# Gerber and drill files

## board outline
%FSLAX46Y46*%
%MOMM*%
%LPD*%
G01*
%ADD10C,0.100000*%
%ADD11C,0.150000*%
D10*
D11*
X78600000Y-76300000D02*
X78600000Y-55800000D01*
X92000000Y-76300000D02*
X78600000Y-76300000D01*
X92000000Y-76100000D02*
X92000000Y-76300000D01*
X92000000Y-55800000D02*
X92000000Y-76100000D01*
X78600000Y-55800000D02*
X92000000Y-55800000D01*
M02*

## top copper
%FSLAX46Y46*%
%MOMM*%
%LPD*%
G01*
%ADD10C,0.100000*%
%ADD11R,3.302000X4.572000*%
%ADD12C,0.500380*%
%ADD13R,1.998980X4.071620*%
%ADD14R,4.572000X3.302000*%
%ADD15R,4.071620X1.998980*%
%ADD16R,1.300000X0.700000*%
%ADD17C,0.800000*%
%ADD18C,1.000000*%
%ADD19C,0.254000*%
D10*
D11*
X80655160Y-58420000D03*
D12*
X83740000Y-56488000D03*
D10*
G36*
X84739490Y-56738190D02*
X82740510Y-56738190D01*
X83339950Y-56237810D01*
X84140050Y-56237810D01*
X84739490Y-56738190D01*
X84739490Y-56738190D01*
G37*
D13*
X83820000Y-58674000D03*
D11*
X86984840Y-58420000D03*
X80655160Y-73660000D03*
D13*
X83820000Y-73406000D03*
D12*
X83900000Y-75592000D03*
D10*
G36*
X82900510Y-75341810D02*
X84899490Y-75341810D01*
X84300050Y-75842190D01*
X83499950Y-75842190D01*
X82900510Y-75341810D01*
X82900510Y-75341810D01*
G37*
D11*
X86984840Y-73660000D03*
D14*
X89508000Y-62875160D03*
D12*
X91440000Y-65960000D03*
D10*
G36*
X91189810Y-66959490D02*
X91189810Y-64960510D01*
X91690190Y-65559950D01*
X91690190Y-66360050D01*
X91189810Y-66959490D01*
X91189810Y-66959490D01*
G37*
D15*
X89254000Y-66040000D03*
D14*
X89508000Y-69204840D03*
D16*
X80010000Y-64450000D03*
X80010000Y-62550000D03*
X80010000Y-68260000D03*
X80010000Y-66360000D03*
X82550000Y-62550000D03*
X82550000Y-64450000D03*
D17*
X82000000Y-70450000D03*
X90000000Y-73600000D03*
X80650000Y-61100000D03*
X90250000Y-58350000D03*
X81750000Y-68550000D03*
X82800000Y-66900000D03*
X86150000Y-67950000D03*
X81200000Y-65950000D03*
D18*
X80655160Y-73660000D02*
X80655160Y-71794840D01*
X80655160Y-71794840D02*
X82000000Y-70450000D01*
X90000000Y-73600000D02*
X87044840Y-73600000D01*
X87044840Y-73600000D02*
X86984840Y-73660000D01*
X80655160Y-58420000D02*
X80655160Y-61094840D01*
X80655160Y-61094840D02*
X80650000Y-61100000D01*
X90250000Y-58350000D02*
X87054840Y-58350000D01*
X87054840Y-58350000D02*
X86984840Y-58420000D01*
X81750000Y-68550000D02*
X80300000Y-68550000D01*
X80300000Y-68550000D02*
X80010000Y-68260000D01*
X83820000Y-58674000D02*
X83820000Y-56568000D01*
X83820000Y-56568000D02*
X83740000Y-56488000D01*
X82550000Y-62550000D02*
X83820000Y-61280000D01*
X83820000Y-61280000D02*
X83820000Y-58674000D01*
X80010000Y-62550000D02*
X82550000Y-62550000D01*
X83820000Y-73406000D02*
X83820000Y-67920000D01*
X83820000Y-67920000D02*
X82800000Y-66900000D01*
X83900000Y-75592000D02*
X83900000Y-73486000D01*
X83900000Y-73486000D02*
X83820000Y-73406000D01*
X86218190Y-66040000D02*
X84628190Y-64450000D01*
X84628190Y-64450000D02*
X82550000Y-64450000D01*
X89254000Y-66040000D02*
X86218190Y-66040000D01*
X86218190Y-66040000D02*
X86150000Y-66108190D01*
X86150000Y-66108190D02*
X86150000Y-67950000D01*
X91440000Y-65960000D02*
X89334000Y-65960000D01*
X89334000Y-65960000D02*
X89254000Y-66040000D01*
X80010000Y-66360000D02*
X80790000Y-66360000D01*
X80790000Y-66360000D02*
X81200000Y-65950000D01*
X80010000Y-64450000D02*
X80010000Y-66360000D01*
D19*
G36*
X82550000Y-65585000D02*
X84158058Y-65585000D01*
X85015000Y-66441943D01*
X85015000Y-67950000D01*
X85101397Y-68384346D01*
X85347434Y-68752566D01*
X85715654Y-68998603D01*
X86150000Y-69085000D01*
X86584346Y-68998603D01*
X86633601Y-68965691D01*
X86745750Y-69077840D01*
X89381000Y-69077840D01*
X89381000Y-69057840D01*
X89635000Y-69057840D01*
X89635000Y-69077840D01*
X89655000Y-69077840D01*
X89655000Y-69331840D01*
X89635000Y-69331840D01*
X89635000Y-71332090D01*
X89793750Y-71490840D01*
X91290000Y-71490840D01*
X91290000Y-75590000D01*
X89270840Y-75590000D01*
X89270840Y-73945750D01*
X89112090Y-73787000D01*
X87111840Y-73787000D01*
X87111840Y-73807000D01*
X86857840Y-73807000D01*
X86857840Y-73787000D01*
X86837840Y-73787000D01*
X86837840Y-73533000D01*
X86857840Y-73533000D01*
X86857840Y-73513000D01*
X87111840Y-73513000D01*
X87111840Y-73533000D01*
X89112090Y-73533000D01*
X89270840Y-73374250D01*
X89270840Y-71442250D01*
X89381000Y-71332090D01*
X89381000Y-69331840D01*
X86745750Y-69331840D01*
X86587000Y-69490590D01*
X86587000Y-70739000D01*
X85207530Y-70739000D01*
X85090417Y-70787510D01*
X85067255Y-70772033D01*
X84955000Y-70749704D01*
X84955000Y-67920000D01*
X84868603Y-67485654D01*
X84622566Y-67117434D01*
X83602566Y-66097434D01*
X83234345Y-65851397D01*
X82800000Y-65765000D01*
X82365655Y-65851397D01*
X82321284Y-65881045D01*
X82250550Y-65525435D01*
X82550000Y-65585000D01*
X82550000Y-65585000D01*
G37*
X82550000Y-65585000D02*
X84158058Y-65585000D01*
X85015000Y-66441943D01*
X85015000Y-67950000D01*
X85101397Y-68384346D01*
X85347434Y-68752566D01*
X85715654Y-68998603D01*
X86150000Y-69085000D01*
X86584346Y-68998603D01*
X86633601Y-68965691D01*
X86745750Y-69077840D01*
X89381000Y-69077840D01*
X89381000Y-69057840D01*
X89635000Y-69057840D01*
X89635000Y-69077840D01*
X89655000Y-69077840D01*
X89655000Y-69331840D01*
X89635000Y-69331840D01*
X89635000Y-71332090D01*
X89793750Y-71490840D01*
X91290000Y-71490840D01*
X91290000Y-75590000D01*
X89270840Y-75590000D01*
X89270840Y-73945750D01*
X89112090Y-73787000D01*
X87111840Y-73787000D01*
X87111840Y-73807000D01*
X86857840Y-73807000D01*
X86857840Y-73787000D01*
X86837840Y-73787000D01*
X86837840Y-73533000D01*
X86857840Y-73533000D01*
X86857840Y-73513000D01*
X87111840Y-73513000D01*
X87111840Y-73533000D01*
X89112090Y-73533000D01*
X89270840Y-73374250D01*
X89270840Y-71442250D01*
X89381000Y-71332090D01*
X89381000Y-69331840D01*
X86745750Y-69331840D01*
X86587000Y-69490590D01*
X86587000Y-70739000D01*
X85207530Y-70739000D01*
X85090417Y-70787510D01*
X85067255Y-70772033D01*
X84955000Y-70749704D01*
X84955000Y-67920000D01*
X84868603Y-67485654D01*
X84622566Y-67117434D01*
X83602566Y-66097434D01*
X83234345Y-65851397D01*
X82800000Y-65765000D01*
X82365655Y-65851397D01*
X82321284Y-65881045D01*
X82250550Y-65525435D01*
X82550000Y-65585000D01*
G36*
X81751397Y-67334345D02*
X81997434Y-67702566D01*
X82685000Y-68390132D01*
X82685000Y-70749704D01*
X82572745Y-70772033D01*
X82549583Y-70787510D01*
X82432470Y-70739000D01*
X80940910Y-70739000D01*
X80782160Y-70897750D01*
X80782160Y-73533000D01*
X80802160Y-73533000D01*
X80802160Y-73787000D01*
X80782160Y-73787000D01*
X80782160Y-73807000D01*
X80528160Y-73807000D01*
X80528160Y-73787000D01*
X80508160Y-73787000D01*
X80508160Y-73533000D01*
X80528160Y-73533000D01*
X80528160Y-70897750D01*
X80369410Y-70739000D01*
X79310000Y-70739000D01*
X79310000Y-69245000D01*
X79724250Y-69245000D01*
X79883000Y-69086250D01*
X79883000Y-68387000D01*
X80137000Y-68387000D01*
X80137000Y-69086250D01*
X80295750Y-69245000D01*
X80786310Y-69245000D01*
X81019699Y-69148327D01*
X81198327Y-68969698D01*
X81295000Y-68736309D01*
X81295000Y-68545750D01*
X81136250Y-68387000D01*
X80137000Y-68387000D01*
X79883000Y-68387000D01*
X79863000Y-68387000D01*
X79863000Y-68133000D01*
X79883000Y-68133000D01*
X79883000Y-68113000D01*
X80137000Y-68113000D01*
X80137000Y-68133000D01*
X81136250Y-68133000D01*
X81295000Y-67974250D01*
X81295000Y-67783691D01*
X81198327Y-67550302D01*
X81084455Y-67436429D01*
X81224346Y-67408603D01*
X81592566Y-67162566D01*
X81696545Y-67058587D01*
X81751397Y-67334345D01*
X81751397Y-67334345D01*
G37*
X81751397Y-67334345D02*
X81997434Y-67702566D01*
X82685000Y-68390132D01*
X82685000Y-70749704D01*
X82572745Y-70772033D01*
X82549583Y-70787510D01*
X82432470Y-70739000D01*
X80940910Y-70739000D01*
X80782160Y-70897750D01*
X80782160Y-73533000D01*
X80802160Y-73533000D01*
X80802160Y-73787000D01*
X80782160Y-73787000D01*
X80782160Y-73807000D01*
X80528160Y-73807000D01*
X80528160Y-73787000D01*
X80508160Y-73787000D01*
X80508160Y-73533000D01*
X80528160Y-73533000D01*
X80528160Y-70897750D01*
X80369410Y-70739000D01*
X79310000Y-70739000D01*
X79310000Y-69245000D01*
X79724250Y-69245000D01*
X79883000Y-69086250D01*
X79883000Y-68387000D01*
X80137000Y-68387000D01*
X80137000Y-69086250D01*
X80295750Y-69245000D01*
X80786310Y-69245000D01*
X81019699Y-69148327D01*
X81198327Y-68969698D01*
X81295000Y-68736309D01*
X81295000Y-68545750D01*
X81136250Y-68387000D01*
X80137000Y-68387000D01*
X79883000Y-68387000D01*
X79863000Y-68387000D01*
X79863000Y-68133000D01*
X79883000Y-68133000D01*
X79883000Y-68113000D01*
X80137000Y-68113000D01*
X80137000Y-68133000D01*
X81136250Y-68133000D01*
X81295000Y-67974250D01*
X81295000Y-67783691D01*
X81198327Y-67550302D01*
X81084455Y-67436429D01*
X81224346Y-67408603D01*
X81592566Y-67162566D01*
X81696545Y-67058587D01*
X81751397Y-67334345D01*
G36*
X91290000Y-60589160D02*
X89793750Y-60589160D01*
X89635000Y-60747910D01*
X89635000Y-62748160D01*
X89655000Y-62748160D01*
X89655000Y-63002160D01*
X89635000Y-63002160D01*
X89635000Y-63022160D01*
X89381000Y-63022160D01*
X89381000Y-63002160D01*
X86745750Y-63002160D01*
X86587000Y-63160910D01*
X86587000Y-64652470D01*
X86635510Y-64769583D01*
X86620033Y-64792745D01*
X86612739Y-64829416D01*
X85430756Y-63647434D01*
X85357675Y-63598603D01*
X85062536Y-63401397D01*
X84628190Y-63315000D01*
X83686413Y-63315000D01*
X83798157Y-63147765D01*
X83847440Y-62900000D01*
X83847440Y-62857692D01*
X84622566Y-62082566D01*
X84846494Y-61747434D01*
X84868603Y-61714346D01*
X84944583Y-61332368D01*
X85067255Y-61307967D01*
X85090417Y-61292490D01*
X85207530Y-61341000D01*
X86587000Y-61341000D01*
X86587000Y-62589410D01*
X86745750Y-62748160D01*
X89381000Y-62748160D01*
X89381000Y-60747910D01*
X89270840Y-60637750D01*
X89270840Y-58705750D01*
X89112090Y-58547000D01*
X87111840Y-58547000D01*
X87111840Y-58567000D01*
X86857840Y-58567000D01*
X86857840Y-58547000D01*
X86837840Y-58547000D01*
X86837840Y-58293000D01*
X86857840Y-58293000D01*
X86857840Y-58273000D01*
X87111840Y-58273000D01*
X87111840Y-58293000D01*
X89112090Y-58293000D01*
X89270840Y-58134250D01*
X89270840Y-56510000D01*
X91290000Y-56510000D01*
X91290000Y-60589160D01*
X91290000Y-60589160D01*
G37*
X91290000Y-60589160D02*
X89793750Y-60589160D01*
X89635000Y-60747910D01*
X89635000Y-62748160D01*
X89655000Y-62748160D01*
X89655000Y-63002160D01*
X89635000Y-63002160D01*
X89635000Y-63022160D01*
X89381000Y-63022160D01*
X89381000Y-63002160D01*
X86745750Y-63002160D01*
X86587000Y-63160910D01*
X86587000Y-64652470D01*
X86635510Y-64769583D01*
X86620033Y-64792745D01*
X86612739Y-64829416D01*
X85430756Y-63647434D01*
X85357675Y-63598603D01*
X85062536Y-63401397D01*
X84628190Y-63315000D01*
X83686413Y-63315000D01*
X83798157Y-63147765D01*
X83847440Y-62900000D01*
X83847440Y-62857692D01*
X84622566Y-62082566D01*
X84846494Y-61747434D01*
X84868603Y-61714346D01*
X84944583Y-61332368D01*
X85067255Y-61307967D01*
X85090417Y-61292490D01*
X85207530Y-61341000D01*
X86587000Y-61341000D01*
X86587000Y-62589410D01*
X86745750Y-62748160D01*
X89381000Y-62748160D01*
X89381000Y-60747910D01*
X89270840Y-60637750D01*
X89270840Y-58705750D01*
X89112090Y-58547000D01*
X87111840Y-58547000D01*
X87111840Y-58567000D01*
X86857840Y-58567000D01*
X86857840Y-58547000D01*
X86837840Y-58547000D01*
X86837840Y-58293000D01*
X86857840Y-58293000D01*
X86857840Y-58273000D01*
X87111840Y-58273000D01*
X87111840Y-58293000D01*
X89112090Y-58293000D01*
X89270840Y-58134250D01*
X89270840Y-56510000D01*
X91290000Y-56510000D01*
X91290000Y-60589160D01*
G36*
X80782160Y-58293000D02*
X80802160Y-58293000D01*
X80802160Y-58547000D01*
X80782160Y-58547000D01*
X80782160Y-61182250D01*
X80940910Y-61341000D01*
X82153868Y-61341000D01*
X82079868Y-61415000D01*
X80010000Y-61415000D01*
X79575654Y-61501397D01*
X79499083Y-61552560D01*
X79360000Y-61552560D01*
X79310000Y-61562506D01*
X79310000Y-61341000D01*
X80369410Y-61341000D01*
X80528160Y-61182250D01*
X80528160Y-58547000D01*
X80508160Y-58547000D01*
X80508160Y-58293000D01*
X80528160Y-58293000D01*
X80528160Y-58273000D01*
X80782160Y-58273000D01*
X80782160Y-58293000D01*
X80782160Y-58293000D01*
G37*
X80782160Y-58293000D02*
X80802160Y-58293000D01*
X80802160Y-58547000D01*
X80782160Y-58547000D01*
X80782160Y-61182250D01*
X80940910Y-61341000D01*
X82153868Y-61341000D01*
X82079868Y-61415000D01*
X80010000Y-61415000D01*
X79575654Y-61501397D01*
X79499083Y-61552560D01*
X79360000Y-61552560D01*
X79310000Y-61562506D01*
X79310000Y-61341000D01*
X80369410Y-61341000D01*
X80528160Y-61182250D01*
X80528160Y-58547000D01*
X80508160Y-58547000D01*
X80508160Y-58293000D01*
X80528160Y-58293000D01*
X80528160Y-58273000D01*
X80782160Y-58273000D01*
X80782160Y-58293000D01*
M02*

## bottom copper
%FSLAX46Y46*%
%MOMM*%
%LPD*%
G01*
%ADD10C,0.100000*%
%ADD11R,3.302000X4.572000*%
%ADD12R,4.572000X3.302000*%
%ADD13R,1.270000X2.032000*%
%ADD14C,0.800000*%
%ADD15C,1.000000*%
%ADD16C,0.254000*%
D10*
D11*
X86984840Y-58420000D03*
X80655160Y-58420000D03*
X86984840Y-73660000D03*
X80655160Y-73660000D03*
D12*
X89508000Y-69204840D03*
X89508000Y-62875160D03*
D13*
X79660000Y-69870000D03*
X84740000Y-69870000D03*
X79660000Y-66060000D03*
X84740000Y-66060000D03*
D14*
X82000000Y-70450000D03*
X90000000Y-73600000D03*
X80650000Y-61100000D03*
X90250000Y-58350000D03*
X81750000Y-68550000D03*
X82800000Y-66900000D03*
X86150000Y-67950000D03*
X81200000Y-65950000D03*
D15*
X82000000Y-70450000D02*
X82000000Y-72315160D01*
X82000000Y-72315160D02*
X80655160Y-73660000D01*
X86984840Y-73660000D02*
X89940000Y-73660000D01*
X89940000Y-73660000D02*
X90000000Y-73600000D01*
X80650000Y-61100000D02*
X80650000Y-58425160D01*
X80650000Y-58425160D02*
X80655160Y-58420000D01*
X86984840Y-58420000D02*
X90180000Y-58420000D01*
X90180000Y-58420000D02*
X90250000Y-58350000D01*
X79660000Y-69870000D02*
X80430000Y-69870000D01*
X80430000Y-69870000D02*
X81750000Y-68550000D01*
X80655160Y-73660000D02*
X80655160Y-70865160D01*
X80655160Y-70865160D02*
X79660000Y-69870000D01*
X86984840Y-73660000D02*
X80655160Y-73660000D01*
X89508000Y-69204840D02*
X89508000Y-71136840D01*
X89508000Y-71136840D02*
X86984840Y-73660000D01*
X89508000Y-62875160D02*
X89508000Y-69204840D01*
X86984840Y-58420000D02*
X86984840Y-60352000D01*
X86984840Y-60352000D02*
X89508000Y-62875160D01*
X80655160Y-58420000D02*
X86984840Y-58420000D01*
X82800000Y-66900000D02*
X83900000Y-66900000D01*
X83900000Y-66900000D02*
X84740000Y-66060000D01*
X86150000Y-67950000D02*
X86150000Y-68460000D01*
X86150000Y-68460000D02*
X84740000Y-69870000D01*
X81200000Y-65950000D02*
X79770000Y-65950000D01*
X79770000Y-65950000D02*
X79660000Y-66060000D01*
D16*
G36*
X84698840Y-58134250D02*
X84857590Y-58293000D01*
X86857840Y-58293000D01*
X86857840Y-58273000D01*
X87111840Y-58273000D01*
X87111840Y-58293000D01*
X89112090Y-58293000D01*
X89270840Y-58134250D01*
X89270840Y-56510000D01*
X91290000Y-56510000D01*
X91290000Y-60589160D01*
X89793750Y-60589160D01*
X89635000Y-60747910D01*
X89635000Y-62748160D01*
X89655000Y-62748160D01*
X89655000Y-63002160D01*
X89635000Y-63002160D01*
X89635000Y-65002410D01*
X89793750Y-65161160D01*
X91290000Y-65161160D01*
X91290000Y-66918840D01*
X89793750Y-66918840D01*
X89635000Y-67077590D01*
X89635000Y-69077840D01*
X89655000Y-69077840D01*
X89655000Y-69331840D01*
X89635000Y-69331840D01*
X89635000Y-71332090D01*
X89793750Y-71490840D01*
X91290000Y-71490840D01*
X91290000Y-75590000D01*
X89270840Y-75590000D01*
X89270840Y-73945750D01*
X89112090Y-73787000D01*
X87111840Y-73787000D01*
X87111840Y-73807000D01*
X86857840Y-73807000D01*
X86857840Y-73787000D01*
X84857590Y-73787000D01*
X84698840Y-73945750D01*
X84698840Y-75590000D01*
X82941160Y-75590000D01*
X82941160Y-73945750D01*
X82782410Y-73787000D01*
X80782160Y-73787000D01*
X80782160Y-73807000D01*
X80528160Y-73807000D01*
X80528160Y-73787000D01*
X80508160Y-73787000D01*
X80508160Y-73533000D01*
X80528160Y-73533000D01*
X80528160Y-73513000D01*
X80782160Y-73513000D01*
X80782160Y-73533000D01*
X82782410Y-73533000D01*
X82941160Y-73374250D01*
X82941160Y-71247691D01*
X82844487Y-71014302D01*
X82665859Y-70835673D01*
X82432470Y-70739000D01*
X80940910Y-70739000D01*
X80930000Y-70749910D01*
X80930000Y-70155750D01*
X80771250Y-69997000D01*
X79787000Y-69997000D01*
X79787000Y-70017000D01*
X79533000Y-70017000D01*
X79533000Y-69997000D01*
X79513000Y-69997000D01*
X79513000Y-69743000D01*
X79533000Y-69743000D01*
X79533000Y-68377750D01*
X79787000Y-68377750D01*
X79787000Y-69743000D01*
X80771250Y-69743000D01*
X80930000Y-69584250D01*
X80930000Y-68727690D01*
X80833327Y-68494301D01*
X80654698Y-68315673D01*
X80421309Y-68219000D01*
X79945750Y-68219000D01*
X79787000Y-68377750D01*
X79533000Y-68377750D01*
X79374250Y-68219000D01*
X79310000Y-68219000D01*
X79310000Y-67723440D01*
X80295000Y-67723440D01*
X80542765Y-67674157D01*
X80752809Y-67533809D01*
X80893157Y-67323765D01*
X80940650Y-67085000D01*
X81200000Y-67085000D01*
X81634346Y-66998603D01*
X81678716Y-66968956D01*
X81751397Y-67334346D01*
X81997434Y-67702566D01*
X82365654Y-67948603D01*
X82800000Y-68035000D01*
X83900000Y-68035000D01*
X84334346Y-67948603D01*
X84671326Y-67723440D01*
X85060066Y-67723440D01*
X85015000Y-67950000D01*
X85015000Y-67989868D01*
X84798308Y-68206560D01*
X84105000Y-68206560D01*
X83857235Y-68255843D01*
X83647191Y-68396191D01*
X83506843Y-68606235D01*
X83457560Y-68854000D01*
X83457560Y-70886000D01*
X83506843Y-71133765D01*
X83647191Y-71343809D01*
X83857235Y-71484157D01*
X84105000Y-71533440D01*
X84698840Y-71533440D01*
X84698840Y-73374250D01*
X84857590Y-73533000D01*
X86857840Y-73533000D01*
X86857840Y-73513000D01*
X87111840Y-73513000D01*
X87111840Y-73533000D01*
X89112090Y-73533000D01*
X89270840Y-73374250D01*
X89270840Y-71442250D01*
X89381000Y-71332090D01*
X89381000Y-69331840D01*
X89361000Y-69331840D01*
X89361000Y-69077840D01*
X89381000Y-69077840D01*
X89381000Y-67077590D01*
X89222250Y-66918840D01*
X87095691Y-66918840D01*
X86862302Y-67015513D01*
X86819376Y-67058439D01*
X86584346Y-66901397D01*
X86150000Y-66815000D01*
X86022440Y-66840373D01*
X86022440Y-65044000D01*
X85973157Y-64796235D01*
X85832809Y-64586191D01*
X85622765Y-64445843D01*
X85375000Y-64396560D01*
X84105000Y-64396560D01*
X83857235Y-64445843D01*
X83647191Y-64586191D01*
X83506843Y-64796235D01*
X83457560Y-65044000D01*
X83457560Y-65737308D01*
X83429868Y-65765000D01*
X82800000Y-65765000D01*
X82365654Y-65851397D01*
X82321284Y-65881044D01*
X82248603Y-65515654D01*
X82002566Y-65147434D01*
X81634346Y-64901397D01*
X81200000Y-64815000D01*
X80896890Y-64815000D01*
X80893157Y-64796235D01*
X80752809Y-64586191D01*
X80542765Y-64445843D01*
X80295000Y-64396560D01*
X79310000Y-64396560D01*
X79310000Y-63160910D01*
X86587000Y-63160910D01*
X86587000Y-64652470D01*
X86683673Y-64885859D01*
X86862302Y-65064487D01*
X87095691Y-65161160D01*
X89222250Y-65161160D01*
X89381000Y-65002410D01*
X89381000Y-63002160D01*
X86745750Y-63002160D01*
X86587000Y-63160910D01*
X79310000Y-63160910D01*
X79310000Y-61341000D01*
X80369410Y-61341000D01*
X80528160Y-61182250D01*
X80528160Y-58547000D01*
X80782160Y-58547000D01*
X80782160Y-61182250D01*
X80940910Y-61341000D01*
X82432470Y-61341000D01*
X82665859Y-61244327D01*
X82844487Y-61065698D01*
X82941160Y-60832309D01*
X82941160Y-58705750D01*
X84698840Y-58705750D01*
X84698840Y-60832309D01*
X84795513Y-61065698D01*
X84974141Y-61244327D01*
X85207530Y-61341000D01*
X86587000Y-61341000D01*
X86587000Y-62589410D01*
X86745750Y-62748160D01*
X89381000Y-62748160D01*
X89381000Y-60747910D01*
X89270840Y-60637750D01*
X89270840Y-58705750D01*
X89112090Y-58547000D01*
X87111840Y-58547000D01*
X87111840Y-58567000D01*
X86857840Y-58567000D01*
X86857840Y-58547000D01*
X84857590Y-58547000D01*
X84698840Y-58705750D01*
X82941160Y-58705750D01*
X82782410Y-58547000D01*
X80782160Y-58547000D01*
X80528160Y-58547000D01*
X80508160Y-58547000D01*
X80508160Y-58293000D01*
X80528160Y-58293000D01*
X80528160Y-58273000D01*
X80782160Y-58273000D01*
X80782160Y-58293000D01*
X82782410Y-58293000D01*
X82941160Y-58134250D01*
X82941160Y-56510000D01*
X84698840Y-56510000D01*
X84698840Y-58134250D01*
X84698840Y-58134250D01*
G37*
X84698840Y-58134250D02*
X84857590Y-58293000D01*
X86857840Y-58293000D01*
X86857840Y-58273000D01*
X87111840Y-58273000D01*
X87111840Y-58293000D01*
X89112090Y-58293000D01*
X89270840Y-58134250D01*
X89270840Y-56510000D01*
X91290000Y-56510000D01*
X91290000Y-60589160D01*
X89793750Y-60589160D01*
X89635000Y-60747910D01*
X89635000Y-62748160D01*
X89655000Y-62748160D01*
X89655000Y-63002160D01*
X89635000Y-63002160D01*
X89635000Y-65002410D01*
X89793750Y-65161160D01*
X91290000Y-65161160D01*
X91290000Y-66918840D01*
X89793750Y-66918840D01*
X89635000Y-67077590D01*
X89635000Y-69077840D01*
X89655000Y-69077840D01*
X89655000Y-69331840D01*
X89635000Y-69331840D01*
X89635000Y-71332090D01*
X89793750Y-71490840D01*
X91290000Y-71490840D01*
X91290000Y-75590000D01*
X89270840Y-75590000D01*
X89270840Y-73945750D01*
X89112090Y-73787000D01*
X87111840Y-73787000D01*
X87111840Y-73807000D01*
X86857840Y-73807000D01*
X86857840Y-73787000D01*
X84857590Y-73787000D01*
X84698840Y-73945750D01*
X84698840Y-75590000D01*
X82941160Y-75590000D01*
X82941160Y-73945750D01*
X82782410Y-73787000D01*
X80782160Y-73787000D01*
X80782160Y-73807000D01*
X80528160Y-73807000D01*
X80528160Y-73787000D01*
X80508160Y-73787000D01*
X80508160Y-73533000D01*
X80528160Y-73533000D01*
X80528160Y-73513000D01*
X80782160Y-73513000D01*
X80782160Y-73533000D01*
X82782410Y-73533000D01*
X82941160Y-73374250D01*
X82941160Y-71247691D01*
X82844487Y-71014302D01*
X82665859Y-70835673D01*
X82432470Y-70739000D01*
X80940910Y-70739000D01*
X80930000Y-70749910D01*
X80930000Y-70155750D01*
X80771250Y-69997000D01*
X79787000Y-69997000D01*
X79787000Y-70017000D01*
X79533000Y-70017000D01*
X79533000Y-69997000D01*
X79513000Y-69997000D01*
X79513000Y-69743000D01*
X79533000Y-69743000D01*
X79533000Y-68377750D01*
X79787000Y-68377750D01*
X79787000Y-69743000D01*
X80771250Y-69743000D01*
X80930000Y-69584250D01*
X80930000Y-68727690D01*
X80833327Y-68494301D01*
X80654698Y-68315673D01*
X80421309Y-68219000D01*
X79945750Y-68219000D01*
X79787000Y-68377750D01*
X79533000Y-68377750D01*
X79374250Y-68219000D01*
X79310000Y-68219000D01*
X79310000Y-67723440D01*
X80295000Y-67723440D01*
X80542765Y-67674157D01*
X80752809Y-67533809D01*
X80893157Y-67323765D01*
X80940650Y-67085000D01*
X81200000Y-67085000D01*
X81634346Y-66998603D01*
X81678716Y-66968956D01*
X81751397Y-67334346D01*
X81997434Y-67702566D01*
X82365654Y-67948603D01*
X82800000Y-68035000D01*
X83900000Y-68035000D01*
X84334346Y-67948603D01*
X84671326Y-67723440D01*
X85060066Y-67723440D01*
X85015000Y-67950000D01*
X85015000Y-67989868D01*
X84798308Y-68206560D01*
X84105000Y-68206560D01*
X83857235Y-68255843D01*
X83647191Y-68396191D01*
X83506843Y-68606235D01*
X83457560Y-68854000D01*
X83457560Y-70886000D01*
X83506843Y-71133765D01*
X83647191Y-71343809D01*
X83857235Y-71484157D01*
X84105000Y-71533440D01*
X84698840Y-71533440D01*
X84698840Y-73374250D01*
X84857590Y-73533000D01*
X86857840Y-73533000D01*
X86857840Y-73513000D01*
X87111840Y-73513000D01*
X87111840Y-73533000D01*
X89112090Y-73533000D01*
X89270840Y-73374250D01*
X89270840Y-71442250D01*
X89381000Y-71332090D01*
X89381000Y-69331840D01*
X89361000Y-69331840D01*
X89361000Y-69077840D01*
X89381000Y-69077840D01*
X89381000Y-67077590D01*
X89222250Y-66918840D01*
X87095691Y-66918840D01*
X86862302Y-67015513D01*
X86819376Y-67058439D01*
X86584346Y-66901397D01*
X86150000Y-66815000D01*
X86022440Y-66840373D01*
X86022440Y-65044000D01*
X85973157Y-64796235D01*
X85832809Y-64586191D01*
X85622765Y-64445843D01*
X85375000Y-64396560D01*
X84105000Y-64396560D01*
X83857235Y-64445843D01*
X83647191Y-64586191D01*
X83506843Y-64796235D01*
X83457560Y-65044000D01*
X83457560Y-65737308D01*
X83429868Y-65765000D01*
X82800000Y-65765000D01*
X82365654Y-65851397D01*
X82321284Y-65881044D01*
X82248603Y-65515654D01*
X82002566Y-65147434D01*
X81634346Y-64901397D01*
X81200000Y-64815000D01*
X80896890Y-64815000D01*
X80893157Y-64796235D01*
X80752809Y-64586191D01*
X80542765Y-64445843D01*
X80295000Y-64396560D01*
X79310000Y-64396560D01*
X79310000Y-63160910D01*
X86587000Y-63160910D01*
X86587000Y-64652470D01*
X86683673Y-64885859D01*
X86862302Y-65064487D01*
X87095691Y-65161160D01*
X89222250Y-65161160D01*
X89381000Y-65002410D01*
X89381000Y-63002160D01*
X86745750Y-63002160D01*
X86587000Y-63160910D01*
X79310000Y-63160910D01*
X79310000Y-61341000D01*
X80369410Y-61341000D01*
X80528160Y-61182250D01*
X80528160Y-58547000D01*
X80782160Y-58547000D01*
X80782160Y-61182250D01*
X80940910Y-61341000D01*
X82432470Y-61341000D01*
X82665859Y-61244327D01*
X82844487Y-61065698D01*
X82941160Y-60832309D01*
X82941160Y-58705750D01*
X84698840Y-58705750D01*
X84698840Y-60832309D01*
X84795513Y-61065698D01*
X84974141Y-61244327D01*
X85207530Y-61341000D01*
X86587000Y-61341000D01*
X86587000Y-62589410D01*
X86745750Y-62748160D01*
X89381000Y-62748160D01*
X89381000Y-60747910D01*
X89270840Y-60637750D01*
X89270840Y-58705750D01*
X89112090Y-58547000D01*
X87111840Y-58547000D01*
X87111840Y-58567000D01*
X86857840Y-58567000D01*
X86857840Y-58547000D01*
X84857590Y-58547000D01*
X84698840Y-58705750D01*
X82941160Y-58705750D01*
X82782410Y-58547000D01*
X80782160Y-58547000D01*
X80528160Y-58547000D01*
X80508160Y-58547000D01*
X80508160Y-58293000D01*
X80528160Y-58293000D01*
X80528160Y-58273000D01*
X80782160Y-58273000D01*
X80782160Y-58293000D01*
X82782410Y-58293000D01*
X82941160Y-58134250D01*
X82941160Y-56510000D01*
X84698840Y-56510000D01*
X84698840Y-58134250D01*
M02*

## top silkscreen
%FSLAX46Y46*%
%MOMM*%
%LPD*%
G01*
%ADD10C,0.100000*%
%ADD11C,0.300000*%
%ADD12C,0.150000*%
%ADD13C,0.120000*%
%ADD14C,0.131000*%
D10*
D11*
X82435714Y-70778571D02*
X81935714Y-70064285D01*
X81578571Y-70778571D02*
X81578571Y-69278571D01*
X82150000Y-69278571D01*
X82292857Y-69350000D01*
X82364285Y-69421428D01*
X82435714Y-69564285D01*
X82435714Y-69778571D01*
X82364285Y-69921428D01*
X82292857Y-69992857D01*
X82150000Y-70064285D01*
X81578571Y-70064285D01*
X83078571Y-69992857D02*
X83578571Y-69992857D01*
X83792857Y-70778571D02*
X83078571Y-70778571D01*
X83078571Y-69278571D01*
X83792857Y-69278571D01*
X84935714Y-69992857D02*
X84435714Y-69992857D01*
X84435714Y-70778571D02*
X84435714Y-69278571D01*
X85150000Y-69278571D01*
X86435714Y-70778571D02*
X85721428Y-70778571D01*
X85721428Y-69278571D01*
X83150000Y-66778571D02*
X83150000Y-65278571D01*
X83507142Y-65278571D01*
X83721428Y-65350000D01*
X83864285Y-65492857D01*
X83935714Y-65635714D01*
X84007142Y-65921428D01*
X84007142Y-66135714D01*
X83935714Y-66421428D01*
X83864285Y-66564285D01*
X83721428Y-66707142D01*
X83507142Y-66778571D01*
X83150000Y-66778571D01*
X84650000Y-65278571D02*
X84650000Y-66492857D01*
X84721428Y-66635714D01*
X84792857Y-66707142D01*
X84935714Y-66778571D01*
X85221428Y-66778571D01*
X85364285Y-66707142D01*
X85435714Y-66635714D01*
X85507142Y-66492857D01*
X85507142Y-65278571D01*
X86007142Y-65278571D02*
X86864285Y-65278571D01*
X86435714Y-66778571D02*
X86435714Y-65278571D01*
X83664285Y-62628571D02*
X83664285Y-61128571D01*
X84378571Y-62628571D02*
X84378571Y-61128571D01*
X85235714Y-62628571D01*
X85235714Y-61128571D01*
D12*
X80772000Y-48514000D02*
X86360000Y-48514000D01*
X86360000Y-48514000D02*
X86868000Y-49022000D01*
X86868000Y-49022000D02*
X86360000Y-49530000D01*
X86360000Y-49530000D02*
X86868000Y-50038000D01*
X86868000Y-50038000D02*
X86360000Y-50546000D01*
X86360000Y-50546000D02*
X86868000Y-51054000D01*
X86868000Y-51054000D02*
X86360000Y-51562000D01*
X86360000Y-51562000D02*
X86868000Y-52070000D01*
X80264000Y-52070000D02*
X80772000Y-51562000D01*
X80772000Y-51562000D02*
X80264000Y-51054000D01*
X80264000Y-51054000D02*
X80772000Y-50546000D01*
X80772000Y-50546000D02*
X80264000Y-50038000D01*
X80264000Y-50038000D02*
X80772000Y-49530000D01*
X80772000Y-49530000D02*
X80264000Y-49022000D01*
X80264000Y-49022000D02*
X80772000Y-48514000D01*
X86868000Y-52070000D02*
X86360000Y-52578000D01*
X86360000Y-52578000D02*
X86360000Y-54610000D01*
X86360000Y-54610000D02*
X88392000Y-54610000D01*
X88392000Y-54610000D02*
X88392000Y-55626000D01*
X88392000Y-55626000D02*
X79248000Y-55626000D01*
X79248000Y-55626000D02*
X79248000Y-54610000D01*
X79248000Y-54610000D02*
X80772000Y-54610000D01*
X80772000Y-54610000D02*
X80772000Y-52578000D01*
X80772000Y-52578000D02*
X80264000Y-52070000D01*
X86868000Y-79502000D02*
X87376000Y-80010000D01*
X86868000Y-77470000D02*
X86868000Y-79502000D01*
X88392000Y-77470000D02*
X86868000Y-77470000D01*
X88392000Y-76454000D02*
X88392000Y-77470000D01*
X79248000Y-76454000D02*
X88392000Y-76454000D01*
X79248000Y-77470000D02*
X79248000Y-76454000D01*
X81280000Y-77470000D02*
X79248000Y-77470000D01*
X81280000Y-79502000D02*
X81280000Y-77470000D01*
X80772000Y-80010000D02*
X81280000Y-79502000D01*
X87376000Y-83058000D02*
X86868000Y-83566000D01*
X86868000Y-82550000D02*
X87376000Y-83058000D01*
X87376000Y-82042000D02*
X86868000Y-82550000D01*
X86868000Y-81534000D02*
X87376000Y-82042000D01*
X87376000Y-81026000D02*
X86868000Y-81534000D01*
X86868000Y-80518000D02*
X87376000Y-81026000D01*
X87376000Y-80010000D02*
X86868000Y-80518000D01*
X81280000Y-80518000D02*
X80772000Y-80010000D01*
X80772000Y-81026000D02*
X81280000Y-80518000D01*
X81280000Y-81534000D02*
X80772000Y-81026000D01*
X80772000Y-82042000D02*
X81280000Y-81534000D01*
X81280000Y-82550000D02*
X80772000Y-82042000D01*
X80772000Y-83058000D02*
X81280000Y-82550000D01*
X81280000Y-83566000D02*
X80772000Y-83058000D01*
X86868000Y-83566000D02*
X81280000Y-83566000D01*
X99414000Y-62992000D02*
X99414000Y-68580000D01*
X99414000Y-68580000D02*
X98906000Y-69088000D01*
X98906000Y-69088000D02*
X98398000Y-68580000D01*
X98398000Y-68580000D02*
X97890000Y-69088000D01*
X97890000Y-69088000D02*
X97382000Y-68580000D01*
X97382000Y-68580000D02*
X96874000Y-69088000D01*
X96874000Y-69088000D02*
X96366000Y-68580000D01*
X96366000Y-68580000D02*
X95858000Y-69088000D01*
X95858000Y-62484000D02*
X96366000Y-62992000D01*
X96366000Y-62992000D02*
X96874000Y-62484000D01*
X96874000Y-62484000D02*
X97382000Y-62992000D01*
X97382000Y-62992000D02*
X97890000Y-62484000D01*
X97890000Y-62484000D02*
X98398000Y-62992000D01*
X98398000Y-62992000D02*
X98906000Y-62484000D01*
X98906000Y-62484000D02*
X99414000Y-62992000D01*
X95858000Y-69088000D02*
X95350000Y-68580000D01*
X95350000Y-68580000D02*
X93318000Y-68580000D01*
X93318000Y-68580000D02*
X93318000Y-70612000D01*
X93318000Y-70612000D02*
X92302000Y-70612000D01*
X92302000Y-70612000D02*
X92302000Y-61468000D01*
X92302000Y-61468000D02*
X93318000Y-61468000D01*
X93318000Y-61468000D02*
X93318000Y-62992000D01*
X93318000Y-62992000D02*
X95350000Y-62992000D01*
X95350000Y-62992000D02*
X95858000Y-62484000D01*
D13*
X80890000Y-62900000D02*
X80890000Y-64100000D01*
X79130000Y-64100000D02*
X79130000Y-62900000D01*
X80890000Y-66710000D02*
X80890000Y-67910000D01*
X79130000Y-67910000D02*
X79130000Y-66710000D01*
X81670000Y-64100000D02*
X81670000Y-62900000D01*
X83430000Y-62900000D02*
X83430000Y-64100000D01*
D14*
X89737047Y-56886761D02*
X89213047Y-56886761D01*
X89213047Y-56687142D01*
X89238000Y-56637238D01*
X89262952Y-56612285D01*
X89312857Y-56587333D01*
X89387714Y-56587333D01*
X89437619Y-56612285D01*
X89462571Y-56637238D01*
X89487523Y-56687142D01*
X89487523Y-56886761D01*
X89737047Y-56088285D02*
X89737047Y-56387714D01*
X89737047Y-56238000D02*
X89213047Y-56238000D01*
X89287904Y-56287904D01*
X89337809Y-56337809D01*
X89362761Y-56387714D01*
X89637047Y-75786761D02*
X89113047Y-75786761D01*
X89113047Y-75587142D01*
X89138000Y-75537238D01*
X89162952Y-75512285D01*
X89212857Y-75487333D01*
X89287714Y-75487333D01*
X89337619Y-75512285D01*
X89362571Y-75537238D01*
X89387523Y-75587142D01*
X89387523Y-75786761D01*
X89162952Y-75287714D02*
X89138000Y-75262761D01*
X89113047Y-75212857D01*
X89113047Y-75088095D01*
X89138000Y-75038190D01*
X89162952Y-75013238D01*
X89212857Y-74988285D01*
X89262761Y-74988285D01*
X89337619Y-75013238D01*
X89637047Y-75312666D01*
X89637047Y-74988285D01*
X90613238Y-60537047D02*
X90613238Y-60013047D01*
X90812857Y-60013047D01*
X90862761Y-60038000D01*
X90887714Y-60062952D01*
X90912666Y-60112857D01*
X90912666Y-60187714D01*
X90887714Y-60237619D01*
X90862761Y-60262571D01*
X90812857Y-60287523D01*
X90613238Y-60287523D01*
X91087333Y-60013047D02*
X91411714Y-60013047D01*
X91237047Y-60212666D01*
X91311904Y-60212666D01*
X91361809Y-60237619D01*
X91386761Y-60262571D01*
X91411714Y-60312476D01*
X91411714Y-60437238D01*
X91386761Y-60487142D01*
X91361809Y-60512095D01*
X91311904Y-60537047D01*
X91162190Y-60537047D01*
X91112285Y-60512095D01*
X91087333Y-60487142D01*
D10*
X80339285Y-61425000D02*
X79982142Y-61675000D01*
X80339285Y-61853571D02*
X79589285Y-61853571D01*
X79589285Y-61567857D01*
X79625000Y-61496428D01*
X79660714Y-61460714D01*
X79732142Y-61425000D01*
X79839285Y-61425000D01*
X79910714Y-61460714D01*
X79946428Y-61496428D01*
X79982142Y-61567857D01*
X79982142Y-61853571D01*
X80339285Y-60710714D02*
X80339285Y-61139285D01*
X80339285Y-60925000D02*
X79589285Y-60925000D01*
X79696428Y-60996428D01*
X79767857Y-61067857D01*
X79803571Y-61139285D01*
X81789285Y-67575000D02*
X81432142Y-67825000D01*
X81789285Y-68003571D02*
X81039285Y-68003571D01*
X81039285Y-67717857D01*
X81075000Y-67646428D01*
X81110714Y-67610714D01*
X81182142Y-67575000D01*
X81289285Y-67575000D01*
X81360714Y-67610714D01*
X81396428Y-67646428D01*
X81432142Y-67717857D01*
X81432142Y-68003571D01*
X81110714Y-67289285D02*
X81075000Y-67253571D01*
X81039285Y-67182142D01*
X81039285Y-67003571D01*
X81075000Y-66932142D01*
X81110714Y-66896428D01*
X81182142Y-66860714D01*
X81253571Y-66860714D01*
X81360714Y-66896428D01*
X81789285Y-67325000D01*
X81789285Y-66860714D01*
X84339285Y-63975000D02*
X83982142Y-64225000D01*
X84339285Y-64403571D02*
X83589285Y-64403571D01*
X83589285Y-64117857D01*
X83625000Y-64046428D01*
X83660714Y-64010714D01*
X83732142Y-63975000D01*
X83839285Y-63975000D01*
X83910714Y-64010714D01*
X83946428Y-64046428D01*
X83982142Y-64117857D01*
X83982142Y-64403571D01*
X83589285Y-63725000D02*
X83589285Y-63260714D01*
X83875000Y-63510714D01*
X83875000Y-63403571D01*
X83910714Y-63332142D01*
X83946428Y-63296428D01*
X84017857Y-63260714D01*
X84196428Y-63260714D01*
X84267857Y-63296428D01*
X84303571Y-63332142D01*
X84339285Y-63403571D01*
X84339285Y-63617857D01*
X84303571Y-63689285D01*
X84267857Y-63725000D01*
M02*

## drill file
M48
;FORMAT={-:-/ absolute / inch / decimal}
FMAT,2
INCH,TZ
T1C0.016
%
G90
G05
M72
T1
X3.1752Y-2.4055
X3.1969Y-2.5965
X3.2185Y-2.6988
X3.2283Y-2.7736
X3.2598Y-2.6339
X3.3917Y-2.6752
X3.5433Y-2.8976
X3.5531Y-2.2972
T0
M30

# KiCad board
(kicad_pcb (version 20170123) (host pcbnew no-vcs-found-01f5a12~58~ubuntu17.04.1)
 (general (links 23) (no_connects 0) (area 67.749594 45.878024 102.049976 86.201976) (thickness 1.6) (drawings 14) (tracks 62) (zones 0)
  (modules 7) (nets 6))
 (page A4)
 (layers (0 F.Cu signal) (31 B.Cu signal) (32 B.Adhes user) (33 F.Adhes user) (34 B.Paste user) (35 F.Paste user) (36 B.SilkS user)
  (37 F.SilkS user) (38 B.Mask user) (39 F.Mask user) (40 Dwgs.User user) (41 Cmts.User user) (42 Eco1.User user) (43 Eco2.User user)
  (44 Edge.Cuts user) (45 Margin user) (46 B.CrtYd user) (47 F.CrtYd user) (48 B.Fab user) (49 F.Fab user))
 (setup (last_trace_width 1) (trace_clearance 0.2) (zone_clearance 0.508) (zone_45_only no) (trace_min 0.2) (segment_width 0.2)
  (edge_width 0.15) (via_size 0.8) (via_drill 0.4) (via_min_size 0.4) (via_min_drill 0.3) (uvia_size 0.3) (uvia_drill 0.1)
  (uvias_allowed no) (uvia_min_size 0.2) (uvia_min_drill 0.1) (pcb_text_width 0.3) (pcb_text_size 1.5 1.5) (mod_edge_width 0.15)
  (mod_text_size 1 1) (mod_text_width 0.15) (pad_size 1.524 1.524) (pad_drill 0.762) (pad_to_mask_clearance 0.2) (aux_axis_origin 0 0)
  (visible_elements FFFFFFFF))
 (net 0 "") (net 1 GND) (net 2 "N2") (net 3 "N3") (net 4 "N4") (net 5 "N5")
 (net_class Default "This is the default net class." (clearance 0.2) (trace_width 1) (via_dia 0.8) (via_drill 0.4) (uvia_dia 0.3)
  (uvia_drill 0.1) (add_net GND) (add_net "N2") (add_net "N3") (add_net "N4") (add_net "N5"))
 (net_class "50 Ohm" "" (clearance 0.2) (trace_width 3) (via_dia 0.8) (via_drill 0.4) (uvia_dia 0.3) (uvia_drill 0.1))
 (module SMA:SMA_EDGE (layer F.Cu) (at 83.82 49.53 90)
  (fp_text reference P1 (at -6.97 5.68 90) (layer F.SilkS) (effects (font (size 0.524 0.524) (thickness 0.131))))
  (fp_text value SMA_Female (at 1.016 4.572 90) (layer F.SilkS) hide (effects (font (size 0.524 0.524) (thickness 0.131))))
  (fp_line (start 1.016 -3.048) (end 1.016 2.54) (layer F.SilkS) (width 0.15))
  (fp_line (start 1.016 2.54) (end 0.508 3.048) (layer F.SilkS) (width 0.15))
  (fp_line (start 0.508 3.048) (end 0 2.54) (layer F.SilkS) (width 0.15))
  (fp_line (start 0 2.54) (end -0.508 3.048) (layer F.SilkS) (width 0.15))
  (fp_line (start -0.508 3.048) (end -1.016 2.54) (layer F.SilkS) (width 0.15))
  (fp_line (start -1.016 2.54) (end -1.524 3.048) (layer F.SilkS) (width 0.15))
  (fp_line (start -1.524 3.048) (end -2.032 2.54) (layer F.SilkS) (width 0.15))
  (fp_line (start -2.032 2.54) (end -2.54 3.048) (layer F.SilkS) (width 0.15))
  (fp_line (start -2.54 -3.556) (end -2.032 -3.048) (layer F.SilkS) (width 0.15))
  (fp_line (start -2.032 -3.048) (end -1.524 -3.556) (layer F.SilkS) (width 0.15))
  (fp_line (start -1.524 -3.556) (end -1.016 -3.048) (layer F.SilkS) (width 0.15))
  (fp_line (start -1.016 -3.048) (end -0.508 -3.556) (layer F.SilkS) (width 0.15))
  (fp_line (start -0.508 -3.556) (end 0 -3.048) (layer F.SilkS) (width 0.15))
  (fp_line (start 0 -3.048) (end 0.508 -3.556) (layer F.SilkS) (width 0.15))
  (fp_line (start 0.508 -3.556) (end 1.016 -3.048) (layer F.SilkS) (width 0.15))
  (fp_line (start -2.54 3.048) (end -3.048 2.54) (layer F.SilkS) (width 0.15))
  (fp_line (start -3.048 2.54) (end -5.08 2.54) (layer F.SilkS) (width 0.15))
  (fp_line (start -5.08 2.54) (end -5.08 4.572) (layer F.SilkS) (width 0.15))
  (fp_line (start -5.08 4.572) (end -6.096 4.572) (layer F.SilkS) (width 0.15))
  (fp_line (start -6.096 4.572) (end -6.096 -4.572) (layer F.SilkS) (width 0.15))
  (fp_line (start -6.096 -4.572) (end -5.08 -4.572) (layer F.SilkS) (width 0.15))
  (fp_line (start -5.08 -4.572) (end -5.08 -3.048) (layer F.SilkS) (width 0.15))
  (fp_line (start -5.08 -3.048) (end -3.048 -3.048) (layer F.SilkS) (width 0.15))
  (fp_line (start -3.048 -3.048) (end -2.54 -3.556) (layer F.SilkS) (width 0.15))
  (pad 2 connect rect (at -8.89 -3.16484 90) (size 4.572 3.302) (layers F.Cu F.Mask) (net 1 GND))
  (pad 1 connect trapezoid (at -6.958 -0.08 90) (size 0.50038 1.39954) (rect_delta 0.59944 0) (layers F.Cu F.Mask) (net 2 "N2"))
  (pad 2 connect rect (at -8.89 3.16484 90) (size 4.572 3.302) (layers B.Cu B.Mask) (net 1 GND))
  (pad 1 connect rect (at -9.144 0 90) (size 4.07162 1.99898) (layers F.Cu F.Mask) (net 2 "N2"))
  (pad 2 connect rect (at -8.89 -3.16484 90) (size 4.572 3.302) (layers B.Cu B.Mask) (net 1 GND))
  (pad 2 connect rect (at -8.89 3.16484 90) (size 4.572 3.302) (layers F.Cu F.Mask) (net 1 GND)))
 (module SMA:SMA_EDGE (layer F.Cu) (at 83.82 82.55 270)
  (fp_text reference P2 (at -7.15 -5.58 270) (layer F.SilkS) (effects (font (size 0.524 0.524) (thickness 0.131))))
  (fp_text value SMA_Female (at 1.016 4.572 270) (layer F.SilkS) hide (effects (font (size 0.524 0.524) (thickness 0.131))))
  (fp_line (start -3.048 -3.048) (end -2.54 -3.556) (layer F.SilkS) (width 0.15))
  (fp_line (start -5.08 -3.048) (end -3.048 -3.048) (layer F.SilkS) (width 0.15))
  (fp_line (start -5.08 -4.572) (end -5.08 -3.048) (layer F.SilkS) (width 0.15))
  (fp_line (start -6.096 -4.572) (end -5.08 -4.572) (layer F.SilkS) (width 0.15))
  (fp_line (start -6.096 4.572) (end -6.096 -4.572) (layer F.SilkS) (width 0.15))
  (fp_line (start -5.08 4.572) (end -6.096 4.572) (layer F.SilkS) (width 0.15))
  (fp_line (start -5.08 2.54) (end -5.08 4.572) (layer F.SilkS) (width 0.15))
  (fp_line (start -3.048 2.54) (end -5.08 2.54) (layer F.SilkS) (width 0.15))
  (fp_line (start -2.54 3.048) (end -3.048 2.54) (layer F.SilkS) (width 0.15))
  (fp_line (start 0.508 -3.556) (end 1.016 -3.048) (layer F.SilkS) (width 0.15))
  (fp_line (start 0 -3.048) (end 0.508 -3.556) (layer F.SilkS) (width 0.15))
  (fp_line (start -0.508 -3.556) (end 0 -3.048) (layer F.SilkS) (width 0.15))
  (fp_line (start -1.016 -3.048) (end -0.508 -3.556) (layer F.SilkS) (width 0.15))
  (fp_line (start -1.524 -3.556) (end -1.016 -3.048) (layer F.SilkS) (width 0.15))
  (fp_line (start -2.032 -3.048) (end -1.524 -3.556) (layer F.SilkS) (width 0.15))
  (fp_line (start -2.54 -3.556) (end -2.032 -3.048) (layer F.SilkS) (width 0.15))
  (fp_line (start -2.032 2.54) (end -2.54 3.048) (layer F.SilkS) (width 0.15))
  (fp_line (start -1.524 3.048) (end -2.032 2.54) (layer F.SilkS) (width 0.15))
  (fp_line (start -1.016 2.54) (end -1.524 3.048) (layer F.SilkS) (width 0.15))
  (fp_line (start -0.508 3.048) (end -1.016 2.54) (layer F.SilkS) (width 0.15))
  (fp_line (start 0 2.54) (end -0.508 3.048) (layer F.SilkS) (width 0.15))
  (fp_line (start 0.508 3.048) (end 0 2.54) (layer F.SilkS) (width 0.15))
  (fp_line (start 1.016 2.54) (end 0.508 3.048) (layer F.SilkS) (width 0.15))
  (fp_line (start 1.016 -3.048) (end 1.016 2.54) (layer F.SilkS) (width 0.15))
  (pad 2 connect rect (at -8.89 3.16484 270) (size 4.572 3.302) (layers F.Cu F.Mask) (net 1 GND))
  (pad 2 connect rect (at -8.89 -3.16484 270) (size 4.572 3.302) (layers B.Cu B.Mask) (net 1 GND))
  (pad 1 connect rect (at -9.144 0 270) (size 4.07162 1.99898) (layers F.Cu F.Mask) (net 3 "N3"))
  (pad 2 connect rect (at -8.89 3.16484 270) (size 4.572 3.302) (layers B.Cu B.Mask) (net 1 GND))
  (pad 1 connect trapezoid (at -6.958 -0.08 270) (size 0.50038 1.39954) (rect_delta 0.59944 0) (layers F.Cu F.Mask) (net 3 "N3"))
  (pad 2 connect rect (at -8.89 -3.16484 270) (size 4.572 3.302) (layers F.Cu F.Mask) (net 1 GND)))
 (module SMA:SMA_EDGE (layer F.Cu) (at 98.398 66.04)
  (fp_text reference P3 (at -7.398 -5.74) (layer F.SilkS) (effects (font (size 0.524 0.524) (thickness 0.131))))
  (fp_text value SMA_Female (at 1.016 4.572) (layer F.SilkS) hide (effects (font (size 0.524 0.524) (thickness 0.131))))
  (fp_line (start 1.016 -3.048) (end 1.016 2.54) (layer F.SilkS) (width 0.15))
  (fp_line (start 1.016 2.54) (end 0.508 3.048) (layer F.SilkS) (width 0.15))
  (fp_line (start 0.508 3.048) (end 0 2.54) (layer F.SilkS) (width 0.15))
  (fp_line (start 0 2.54) (end -0.508 3.048) (layer F.SilkS) (width 0.15))
  (fp_line (start -0.508 3.048) (end -1.016 2.54) (layer F.SilkS) (width 0.15))
  (fp_line (start -1.016 2.54) (end -1.524 3.048) (layer F.SilkS) (width 0.15))
  (fp_line (start -1.524 3.048) (end -2.032 2.54) (layer F.SilkS) (width 0.15))
  (fp_line (start -2.032 2.54) (end -2.54 3.048) (layer F.SilkS) (width 0.15))
  (fp_line (start -2.54 -3.556) (end -2.032 -3.048) (layer F.SilkS) (width 0.15))
  (fp_line (start -2.032 -3.048) (end -1.524 -3.556) (layer F.SilkS) (width 0.15))
  (fp_line (start -1.524 -3.556) (end -1.016 -3.048) (layer F.SilkS) (width 0.15))
  (fp_line (start -1.016 -3.048) (end -0.508 -3.556) (layer F.SilkS) (width 0.15))
  (fp_line (start -0.508 -3.556) (end 0 -3.048) (layer F.SilkS) (width 0.15))
  (fp_line (start 0 -3.048) (end 0.508 -3.556) (layer F.SilkS) (width 0.15))
  (fp_line (start 0.508 -3.556) (end 1.016 -3.048) (layer F.SilkS) (width 0.15))
  (fp_line (start -2.54 3.048) (end -3.048 2.54) (layer F.SilkS) (width 0.15))
  (fp_line (start -3.048 2.54) (end -5.08 2.54) (layer F.SilkS) (width 0.15))
  (fp_line (start -5.08 2.54) (end -5.08 4.572) (layer F.SilkS) (width 0.15))
  (fp_line (start -5.08 4.572) (end -6.096 4.572) (layer F.SilkS) (width 0.15))
  (fp_line (start -6.096 4.572) (end -6.096 -4.572) (layer F.SilkS) (width 0.15))
  (fp_line (start -6.096 -4.572) (end -5.08 -4.572) (layer F.SilkS) (width 0.15))
  (fp_line (start -5.08 -4.572) (end -5.08 -3.048) (layer F.SilkS) (width 0.15))
  (fp_line (start -5.08 -3.048) (end -3.048 -3.048) (layer F.SilkS) (width 0.15))
  (fp_line (start -3.048 -3.048) (end -2.54 -3.556) (layer F.SilkS) (width 0.15))
  (pad 2 connect rect (at -8.89 -3.16484) (size 4.572 3.302) (layers F.Cu F.Mask) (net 1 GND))
  (pad 1 connect trapezoid (at -6.958 -0.08) (size 0.50038 1.39954) (rect_delta 0.59944 0) (layers F.Cu F.Mask) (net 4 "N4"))
  (pad 2 connect rect (at -8.89 3.16484) (size 4.572 3.302) (layers B.Cu B.Mask) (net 1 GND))
  (pad 1 connect rect (at -9.144 0) (size 4.07162 1.99898) (layers F.Cu F.Mask) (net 4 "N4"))
  (pad 2 connect rect (at -8.89 -3.16484) (size 4.572 3.302) (layers B.Cu B.Mask) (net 1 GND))
  (pad 2 connect rect (at -8.89 3.16484) (size 4.572 3.302) (layers F.Cu F.Mask) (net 1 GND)))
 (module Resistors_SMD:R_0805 (layer F.Cu) (at 80.01 63.5 270)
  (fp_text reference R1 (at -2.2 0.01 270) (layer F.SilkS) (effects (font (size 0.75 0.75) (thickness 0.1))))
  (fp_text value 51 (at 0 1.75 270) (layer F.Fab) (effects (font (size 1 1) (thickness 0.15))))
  (fp_line (start -0.6 -0.88) (end 0.6 -0.88) (layer F.SilkS) (width 0.12))
  (fp_line (start 0.6 0.88) (end -0.6 0.88) (layer F.SilkS) (width 0.12))
  (pad 2 smd rect (at 0.95 0 270) (size 0.7 1.3) (layers F.Cu F.Paste F.Mask) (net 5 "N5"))
  (pad 1 smd rect (at -0.95 0 270) (size 0.7 1.3) (layers F.Cu F.Paste F.Mask) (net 2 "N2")))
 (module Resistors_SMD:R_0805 (layer F.Cu) (at 80.01 67.31 270)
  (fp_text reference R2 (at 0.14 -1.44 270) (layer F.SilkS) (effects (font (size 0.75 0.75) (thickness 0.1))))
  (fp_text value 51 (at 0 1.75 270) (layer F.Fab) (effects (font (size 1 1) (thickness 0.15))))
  (fp_line (start -0.6 -0.88) (end 0.6 -0.88) (layer F.SilkS) (width 0.12))
  (fp_line (start 0.6 0.88) (end -0.6 0.88) (layer F.SilkS) (width 0.12))
  (pad 2 smd rect (at 0.95 0 270) (size 0.7 1.3) (layers F.Cu F.Paste F.Mask) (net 1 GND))
  (pad 1 smd rect (at -0.95 0 270) (size 0.7 1.3) (layers F.Cu F.Paste F.Mask) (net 5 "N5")))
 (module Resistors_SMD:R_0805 (layer F.Cu) (at 82.55 63.5 270)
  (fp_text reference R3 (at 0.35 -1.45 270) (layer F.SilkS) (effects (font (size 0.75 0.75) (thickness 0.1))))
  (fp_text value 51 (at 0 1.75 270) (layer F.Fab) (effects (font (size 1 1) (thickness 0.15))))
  (fp_line (start 0.6 0.88) (end -0.6 0.88) (layer F.SilkS) (width 0.12))
  (fp_line (start -0.6 -0.88) (end 0.6 -0.88) (layer F.SilkS) (width 0.12))
  (pad 1 smd rect (at -0.95 0 270) (size 0.7 1.3) (layers F.Cu F.Paste F.Mask) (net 2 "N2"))
  (pad 2 smd rect (at 0.95 0 270) (size 0.7 1.3) (layers F.Cu F.Paste F.Mask) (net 4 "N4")))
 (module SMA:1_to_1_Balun (layer B.Cu) (at 82.2 68.6)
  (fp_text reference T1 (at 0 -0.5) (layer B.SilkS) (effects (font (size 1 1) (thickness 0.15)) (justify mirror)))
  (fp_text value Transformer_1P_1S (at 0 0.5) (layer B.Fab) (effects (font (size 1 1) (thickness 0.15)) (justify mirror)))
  (pad 1 smd rect (at -2.54 1.27) (size 1.27 2.032) (layers B.Cu B.Paste B.Mask) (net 1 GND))
  (pad 3 smd rect (at 2.54 1.27) (size 1.27 2.032) (layers B.Cu B.Paste B.Mask) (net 4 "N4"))
  (pad 2 smd rect (at -2.54 -2.54) (size 1.27 2.032) (layers B.Cu B.Paste B.Mask) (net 5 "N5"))
  (pad 4 smd rect (at 2.54 -2.54) (size 1.27 2.032) (layers B.Cu B.Paste B.Mask) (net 3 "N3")))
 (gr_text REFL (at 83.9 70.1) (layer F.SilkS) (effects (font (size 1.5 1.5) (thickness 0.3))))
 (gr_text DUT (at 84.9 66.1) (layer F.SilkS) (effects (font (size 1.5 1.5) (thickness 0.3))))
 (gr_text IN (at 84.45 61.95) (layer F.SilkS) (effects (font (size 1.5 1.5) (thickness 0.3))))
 (gr_line (start 78.6 76.3) (end 78.6 55.8) (layer Edge.Cuts) (width 0.15))
 (gr_line (start 92 76.3) (end 78.6 76.3) (layer Edge.Cuts) (width 0.15))
 (gr_line (start 92 76.1) (end 92 76.3) (layer Edge.Cuts) (width 0.15))
 (gr_line (start 92 55.8) (end 92 76.1) (layer Edge.Cuts) (width 0.15))
 (gr_line (start 78.6 55.8) (end 92 55.8) (layer Edge.Cuts) (width 0.15))
 (segment (start 82 70.45) (end 82 72.31516) (width 1) (layer B.Cu) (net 1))
 (segment (start 82 72.31516) (end 80.65516 73.66) (width 1) (layer B.Cu) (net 1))
 (segment (start 80.65516 73.66) (end 80.65516 71.79484) (width 1) (layer F.Cu) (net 1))
 (segment (start 80.65516 71.79484) (end 82 70.45) (width 1) (layer F.Cu) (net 1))
 (via (at 82 70.45) (size 0.8) (drill 0.4) (layers F.Cu B.Cu) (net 1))
 (segment (start 90 73.6) (end 87.04484 73.6) (width 1) (layer F.Cu) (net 1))
 (segment (start 87.04484 73.6) (end 86.98484 73.66) (width 1) (layer F.Cu) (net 1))
 (segment (start 86.98484 73.66) (end 89.94 73.66) (width 1) (layer B.Cu) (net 1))
 (segment (start 89.94 73.66) (end 90 73.6) (width 1) (layer B.Cu) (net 1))
 (via (at 90 73.6) (size 0.8) (drill 0.4) (layers F.Cu B.Cu) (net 1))
 (segment (start 80.65 61.1) (end 80.65 58.42516) (width 1) (layer B.Cu) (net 1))
 (segment (start 80.65 58.42516) (end 80.65516 58.42) (width 1) (layer B.Cu) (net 1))
 (segment (start 80.65516 58.42) (end 80.65516 61.09484) (width 1) (layer F.Cu) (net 1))
 (segment (start 80.65516 61.09484) (end 80.65 61.1) (width 1) (layer F.Cu) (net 1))
 (via (at 80.65 61.1) (size 0.8) (drill 0.4) (layers F.Cu B.Cu) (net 1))
 (segment (start 90.25 58.35) (end 87.05484 58.35) (width 1) (layer F.Cu) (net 1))
 (segment (start 87.05484 58.35) (end 86.98484 58.42) (width 1) (layer F.Cu) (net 1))
 (segment (start 86.98484 58.42) (end 90.18 58.42) (width 1) (layer B.Cu) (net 1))
 (segment (start 90.18 58.42) (end 90.25 58.35) (width 1) (layer B.Cu) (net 1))
 (via (at 90.25 58.35) (size 0.8) (drill 0.4) (layers F.Cu B.Cu) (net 1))
 (segment (start 81.75 68.55) (end 80.3 68.55) (width 1) (layer F.Cu) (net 1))
 (segment (start 80.3 68.55) (end 80.01 68.26) (width 1) (layer F.Cu) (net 1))
 (segment (start 79.66 69.87) (end 80.43 69.87) (width 1) (layer B.Cu) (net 1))
 (segment (start 80.43 69.87) (end 81.75 68.55) (width 1) (layer B.Cu) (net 1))
 (via (at 81.75 68.55) (size 0.8) (drill 0.4) (layers F.Cu B.Cu) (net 1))
 (segment (start 80.65516 73.66) (end 80.65516 70.86516) (width 1) (layer B.Cu) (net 1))
 (segment (start 80.65516 70.86516) (end 79.66 69.87) (width 1) (layer B.Cu) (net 1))
 (segment (start 86.98484 73.66) (end 80.65516 73.66) (width 1) (layer B.Cu) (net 1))
 (segment (start 89.508 69.20484) (end 89.508 71.13684) (width 1) (layer B.Cu) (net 1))
 (segment (start 89.508 71.13684) (end 86.98484 73.66) (width 1) (layer B.Cu) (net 1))
 (segment (start 89.508 62.87516) (end 89.508 69.20484) (width 1) (layer B.Cu) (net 1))
 (segment (start 86.98484 58.42) (end 86.98484 60.352) (width 1) (layer B.Cu) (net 1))
 (segment (start 86.98484 60.352) (end 89.508 62.87516) (width 1) (layer B.Cu) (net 1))
 (segment (start 80.65516 58.42) (end 86.98484 58.42) (width 1) (layer B.Cu) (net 1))
 (segment (start 83.82 58.674) (end 83.82 56.568) (width 1) (layer F.Cu) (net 2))
 (segment (start 83.82 56.568) (end 83.74 56.488) (width 1) (layer F.Cu) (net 2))
 (segment (start 82.55 62.55) (end 83.82 61.28) (width 1) (layer F.Cu) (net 2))
 (segment (start 83.82 61.28) (end 83.82 58.674) (width 1) (layer F.Cu) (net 2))
 (segment (start 80.01 62.55) (end 82.55 62.55) (width 1) (layer F.Cu) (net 2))
 (segment (start 82.8 66.9) (end 83.9 66.9) (width 1) (layer B.Cu) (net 3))
 (segment (start 83.9 66.9) (end 84.74 66.06) (width 1) (layer B.Cu) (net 3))
 (segment (start 83.82 73.406) (end 83.82 67.92) (width 1) (layer F.Cu) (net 3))
 (segment (start 83.82 67.92) (end 82.8 66.9) (width 1) (layer F.Cu) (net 3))
 (via (at 82.8 66.9) (size 0.8) (drill 0.4) (layers F.Cu B.Cu) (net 3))
 (segment (start 83.9 75.592) (end 83.9 73.486) (width 1) (layer F.Cu) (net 3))
 (segment (start 83.9 73.486) (end 83.82 73.406) (width 1) (layer F.Cu) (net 3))
 (segment (start 86.21819 66.04) (end 84.62819 64.45) (width 1) (layer F.Cu) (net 4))
 (segment (start 84.62819 64.45) (end 82.55 64.45) (width 1) (layer F.Cu) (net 4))
 (segment (start 86.15 67.95) (end 86.15 68.46) (width 1) (layer B.Cu) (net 4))
 (segment (start 86.15 68.46) (end 84.74 69.87) (width 1) (layer B.Cu) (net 4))
 (segment (start 89.254 66.04) (end 86.21819 66.04) (width 1) (layer F.Cu) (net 4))
 (segment (start 86.21819 66.04) (end 86.15 66.10819) (width 1) (layer F.Cu) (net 4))
 (segment (start 86.15 66.10819) (end 86.15 67.95) (width 1) (layer F.Cu) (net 4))
 (via (at 86.15 67.95) (size 0.8) (drill 0.4) (layers F.Cu B.Cu) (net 4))
 (segment (start 91.44 65.96) (end 89.334 65.96) (width 1) (layer F.Cu) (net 4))
 (segment (start 89.334 65.96) (end 89.254 66.04) (width 1) (layer F.Cu) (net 4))
 (segment (start 81.2 65.95) (end 79.77 65.95) (width 1) (layer B.Cu) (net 5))
 (segment (start 79.77 65.95) (end 79.66 66.06) (width 1) (layer B.Cu) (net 5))
 (segment (start 80.01 66.36) (end 80.79 66.36) (width 1) (layer F.Cu) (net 5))
 (via (at 81.2 65.95) (size 0.8) (drill 0.4) (layers F.Cu B.Cu) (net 5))
 (segment (start 80.79 66.36) (end 81.2 65.95) (width 1) (layer F.Cu) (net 5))
 (segment (start 80.01 64.45) (end 80.01 66.36) (width 1) (layer F.Cu) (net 5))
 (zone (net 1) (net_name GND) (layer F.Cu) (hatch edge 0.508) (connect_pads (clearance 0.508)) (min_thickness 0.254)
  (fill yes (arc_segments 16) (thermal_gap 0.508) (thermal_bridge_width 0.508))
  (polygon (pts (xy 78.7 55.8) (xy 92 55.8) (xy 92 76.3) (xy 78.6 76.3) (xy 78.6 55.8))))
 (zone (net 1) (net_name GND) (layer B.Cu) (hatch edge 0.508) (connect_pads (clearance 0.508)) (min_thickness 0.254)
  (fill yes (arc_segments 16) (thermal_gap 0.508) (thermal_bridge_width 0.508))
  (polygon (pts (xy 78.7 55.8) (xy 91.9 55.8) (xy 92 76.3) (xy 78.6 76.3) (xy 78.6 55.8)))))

